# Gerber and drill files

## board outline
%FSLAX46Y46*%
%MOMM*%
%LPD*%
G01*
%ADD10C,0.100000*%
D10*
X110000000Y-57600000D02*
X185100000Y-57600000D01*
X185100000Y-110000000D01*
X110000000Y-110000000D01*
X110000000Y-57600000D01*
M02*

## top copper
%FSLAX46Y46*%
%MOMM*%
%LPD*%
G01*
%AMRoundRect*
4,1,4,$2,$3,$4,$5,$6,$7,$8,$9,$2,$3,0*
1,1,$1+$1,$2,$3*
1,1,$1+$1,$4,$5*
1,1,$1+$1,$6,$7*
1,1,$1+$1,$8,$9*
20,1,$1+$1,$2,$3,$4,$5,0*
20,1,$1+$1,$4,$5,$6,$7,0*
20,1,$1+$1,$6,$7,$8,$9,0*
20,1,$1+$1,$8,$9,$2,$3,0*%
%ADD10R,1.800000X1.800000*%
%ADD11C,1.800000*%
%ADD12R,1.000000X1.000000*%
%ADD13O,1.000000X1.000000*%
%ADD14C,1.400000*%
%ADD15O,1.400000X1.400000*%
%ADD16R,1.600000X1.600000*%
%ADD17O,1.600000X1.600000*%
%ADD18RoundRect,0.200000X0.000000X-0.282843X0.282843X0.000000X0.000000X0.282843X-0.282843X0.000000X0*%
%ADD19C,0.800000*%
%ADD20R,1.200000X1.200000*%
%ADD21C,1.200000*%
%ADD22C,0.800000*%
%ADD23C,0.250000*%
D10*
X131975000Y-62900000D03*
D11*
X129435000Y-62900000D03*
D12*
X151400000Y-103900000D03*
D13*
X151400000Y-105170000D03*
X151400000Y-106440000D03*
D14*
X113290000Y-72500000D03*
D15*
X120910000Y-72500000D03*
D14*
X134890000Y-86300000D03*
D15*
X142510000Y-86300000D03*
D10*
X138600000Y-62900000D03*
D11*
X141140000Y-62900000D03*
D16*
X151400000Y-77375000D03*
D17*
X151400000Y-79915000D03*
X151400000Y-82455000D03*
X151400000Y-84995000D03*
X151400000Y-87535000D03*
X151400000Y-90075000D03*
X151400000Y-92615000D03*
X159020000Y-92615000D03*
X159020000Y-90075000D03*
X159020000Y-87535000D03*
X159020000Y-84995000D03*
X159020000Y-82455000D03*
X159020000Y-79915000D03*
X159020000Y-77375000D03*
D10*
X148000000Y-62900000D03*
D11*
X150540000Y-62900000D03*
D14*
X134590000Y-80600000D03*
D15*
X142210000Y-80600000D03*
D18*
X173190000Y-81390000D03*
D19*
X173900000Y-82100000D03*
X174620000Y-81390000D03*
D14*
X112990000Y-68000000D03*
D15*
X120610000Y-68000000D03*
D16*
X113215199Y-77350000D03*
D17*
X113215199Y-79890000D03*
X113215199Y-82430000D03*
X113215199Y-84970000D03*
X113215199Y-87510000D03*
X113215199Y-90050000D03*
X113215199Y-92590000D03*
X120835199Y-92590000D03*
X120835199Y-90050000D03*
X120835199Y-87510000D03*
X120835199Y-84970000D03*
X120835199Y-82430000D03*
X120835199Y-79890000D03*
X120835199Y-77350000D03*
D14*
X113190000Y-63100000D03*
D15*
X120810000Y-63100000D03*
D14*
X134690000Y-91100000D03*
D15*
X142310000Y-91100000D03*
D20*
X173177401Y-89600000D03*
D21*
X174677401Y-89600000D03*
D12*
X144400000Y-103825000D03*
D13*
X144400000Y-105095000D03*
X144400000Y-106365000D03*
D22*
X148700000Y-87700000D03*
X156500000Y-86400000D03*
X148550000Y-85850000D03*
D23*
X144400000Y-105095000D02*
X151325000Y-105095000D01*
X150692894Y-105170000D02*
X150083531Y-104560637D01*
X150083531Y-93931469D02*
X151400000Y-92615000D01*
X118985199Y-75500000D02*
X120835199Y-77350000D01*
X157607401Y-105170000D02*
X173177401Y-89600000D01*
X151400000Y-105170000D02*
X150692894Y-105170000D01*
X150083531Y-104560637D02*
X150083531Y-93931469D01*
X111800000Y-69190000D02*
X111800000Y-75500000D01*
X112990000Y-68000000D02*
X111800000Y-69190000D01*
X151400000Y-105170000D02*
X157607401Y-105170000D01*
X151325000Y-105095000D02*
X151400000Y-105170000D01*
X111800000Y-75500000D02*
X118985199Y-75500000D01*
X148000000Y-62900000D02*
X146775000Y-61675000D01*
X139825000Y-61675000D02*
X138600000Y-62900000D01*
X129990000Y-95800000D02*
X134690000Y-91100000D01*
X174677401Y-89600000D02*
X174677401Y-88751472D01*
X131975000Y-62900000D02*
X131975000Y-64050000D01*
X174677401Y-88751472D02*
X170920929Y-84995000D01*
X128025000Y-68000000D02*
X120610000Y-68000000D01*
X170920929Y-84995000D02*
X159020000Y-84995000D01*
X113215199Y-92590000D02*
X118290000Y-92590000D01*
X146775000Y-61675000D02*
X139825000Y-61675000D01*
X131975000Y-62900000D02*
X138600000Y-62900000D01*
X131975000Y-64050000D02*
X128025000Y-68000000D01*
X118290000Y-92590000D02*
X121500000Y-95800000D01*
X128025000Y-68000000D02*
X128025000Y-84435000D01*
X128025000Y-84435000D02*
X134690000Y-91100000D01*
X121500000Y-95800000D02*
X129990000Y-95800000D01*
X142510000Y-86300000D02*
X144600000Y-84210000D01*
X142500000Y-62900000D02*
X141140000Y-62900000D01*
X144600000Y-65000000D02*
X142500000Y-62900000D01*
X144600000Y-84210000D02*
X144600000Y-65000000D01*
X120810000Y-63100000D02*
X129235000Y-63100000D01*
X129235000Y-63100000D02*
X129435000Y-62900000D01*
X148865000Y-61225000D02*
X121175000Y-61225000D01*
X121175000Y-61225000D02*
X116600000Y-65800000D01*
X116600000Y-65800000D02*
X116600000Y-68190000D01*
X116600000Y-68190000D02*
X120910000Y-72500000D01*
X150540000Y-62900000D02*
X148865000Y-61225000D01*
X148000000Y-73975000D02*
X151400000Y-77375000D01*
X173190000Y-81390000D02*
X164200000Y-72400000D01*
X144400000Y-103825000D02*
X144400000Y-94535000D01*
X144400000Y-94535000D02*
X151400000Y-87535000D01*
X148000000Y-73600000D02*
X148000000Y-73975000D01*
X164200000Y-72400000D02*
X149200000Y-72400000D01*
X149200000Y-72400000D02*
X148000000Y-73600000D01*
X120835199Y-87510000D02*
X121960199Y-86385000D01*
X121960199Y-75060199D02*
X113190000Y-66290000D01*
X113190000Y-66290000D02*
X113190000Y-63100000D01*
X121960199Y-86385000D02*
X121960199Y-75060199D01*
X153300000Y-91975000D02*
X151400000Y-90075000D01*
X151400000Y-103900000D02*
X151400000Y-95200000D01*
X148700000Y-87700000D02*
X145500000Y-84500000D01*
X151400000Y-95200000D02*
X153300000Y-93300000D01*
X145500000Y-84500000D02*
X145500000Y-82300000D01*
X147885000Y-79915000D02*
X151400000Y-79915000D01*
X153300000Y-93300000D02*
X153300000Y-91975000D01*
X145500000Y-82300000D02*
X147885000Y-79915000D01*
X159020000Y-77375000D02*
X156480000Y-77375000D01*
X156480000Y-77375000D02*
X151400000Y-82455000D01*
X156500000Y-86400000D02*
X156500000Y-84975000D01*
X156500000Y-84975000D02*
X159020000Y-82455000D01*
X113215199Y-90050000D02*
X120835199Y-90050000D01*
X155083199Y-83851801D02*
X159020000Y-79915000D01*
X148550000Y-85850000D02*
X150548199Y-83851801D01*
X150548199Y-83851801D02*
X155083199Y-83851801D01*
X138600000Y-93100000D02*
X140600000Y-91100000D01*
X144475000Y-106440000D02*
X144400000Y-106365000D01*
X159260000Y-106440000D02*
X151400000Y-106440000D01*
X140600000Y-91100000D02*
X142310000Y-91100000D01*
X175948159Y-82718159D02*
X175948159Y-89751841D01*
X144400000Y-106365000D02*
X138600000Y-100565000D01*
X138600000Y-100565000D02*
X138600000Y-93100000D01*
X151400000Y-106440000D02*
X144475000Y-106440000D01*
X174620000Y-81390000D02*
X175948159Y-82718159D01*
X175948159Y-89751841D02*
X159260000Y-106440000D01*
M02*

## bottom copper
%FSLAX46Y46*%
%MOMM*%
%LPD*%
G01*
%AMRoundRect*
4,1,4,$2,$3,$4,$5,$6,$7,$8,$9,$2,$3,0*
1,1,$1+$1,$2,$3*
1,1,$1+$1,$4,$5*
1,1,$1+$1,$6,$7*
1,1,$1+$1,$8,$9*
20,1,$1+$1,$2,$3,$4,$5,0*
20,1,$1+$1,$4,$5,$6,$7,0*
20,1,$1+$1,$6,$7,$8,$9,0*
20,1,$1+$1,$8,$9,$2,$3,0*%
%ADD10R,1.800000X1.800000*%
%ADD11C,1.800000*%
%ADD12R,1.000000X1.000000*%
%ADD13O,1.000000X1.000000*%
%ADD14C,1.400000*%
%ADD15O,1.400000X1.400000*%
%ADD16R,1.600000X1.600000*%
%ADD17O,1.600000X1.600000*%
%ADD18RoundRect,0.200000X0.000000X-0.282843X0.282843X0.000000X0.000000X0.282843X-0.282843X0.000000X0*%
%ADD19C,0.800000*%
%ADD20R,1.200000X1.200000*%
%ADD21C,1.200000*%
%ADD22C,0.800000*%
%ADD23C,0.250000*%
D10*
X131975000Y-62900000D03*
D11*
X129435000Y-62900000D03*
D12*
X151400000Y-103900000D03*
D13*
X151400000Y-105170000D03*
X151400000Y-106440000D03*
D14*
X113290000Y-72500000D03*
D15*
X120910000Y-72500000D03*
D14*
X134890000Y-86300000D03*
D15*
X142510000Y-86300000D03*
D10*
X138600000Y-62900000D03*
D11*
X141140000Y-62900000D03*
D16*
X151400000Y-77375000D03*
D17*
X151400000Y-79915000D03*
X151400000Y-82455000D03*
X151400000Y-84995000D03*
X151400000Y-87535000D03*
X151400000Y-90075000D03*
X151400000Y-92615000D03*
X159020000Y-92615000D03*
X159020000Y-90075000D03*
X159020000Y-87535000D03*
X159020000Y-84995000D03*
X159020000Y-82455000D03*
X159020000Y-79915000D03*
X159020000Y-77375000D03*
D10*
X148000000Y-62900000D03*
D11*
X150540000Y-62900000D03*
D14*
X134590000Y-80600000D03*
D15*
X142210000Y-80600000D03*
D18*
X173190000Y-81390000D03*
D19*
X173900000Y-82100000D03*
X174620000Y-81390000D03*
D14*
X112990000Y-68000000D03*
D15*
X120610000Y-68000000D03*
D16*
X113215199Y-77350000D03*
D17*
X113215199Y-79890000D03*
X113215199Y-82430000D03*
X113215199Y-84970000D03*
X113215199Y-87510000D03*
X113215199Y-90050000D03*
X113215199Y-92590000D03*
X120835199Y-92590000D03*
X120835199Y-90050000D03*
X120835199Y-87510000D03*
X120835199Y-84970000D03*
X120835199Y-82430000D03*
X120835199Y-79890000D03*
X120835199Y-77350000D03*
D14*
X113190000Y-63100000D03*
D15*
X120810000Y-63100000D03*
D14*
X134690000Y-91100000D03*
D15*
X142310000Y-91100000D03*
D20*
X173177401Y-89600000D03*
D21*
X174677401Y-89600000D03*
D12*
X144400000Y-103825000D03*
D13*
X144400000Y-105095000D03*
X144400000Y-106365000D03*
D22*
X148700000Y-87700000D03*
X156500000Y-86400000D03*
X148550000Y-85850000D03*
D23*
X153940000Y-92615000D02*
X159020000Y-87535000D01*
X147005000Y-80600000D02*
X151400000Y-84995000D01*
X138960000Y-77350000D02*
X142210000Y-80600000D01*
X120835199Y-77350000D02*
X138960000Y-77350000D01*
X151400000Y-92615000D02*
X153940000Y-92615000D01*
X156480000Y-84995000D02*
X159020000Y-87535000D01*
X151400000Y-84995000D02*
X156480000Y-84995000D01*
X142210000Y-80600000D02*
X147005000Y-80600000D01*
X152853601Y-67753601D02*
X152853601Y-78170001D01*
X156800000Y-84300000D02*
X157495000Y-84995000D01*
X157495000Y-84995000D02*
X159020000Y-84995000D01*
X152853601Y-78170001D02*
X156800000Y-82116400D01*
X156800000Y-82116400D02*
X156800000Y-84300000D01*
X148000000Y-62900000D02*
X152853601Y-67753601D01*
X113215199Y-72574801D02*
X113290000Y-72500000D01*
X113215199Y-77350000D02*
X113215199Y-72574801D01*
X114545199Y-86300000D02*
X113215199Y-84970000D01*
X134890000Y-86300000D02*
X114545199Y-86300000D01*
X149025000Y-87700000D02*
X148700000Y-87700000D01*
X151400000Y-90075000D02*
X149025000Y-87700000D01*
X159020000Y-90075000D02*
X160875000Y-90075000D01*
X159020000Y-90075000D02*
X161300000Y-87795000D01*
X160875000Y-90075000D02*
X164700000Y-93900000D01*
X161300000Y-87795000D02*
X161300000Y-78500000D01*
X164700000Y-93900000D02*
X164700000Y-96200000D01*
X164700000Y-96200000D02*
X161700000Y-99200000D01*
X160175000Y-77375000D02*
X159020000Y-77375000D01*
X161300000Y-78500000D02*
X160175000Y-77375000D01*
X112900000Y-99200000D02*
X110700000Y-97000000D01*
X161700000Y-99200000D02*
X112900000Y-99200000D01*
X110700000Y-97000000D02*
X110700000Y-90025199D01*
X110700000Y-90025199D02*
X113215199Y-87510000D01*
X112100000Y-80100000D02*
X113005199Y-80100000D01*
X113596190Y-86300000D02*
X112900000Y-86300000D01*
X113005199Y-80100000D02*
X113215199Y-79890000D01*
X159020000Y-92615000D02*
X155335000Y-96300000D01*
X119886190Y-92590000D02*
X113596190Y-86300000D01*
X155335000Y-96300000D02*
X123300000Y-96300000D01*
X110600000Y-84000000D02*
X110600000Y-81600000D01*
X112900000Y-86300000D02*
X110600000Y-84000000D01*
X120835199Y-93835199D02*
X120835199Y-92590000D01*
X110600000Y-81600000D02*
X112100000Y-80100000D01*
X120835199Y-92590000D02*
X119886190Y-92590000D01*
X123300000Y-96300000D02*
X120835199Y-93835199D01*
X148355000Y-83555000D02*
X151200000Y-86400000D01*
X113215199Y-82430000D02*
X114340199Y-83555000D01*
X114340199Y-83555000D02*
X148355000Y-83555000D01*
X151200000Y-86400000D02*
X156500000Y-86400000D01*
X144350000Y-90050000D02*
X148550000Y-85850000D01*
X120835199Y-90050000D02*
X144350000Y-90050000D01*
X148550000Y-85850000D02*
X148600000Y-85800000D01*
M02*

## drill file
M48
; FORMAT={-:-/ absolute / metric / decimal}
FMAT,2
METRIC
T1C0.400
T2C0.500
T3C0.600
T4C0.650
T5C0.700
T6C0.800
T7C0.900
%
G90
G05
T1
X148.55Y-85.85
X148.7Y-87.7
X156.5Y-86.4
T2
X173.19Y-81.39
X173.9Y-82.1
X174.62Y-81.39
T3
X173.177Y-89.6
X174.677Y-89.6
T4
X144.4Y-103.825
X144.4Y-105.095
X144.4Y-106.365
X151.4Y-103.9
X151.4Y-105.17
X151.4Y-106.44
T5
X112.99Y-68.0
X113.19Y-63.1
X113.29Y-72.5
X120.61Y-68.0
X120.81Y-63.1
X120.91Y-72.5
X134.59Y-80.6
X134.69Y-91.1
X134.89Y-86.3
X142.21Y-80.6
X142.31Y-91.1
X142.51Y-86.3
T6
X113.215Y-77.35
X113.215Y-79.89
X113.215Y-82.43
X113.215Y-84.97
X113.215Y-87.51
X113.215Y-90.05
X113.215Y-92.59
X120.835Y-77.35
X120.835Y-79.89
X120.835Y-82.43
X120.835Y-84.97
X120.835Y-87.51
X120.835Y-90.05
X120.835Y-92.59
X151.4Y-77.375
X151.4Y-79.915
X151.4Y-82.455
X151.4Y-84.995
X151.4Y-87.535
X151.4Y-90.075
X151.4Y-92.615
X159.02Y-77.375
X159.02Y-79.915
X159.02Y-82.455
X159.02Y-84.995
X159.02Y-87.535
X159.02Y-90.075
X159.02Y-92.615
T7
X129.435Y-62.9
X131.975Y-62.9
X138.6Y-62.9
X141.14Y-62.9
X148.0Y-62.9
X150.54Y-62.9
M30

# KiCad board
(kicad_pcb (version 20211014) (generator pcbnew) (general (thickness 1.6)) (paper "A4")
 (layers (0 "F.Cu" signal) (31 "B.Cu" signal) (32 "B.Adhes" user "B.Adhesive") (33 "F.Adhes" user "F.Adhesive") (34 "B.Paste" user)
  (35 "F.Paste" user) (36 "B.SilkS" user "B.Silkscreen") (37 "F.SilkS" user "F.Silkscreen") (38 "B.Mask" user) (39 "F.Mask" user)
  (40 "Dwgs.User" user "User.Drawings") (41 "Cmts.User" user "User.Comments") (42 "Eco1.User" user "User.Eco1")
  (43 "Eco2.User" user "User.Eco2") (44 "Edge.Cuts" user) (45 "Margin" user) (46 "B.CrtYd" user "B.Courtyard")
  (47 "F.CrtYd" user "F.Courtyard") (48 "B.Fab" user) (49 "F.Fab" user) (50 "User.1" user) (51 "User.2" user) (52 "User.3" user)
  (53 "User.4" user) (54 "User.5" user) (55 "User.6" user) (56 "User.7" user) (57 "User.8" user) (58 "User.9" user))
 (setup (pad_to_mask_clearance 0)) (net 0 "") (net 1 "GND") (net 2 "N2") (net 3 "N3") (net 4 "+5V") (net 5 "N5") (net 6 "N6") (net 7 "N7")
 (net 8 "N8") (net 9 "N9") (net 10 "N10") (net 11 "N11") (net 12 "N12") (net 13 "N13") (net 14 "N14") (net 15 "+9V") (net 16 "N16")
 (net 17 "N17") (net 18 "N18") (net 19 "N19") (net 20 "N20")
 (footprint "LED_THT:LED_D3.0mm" (layer "F.Cu") (at 131.975 62.9 180)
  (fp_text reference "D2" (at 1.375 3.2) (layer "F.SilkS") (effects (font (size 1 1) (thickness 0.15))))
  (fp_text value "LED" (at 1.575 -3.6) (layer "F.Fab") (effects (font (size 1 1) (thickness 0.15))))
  (pad "1" thru_hole rect (at 0 0 180) (size 1.8 1.8) (drill 0.9) (layers *.Cu *.Mask) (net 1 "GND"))
  (pad "2" thru_hole circle (at 2.54 0 180) (size 1.8 1.8) (drill 0.9) (layers *.Cu *.Mask) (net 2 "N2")))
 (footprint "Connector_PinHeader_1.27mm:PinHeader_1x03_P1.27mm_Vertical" (layer "F.Cu") (at 151.4 103.9)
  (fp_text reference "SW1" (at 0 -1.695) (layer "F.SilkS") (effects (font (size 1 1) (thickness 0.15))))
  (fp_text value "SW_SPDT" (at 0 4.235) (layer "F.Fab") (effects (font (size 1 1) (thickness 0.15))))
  (pad "1" thru_hole rect (at 0 0) (size 1 1) (drill 0.65) (layers *.Cu *.Mask) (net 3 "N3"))
  (pad "2" thru_hole oval (at 0 1.27) (size 1 1) (drill 0.65) (layers *.Cu *.Mask) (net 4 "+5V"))
  (pad "3" thru_hole oval (at 0 2.54) (size 1 1) (drill 0.65) (layers *.Cu *.Mask) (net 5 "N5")))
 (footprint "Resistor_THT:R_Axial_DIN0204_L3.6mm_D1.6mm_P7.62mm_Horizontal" (layer "F.Cu") (at 113.29 72.5)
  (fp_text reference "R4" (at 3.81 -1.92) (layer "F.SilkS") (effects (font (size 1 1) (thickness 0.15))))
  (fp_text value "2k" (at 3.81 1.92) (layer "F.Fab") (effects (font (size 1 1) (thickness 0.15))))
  (pad "1" thru_hole circle (at 0 0) (size 1.4 1.4) (drill 0.7) (layers *.Cu *.Mask) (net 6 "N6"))
  (pad "2" thru_hole oval (at 7.62 0) (size 1.4 1.4) (drill 0.7) (layers *.Cu *.Mask) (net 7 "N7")))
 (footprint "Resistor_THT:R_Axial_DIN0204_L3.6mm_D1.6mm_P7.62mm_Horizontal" (layer "F.Cu") (at 134.89 86.3)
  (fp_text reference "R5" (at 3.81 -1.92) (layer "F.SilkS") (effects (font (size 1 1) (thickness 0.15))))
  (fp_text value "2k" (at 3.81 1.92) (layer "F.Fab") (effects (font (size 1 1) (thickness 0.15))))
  (pad "1" thru_hole circle (at 0 0) (size 1.4 1.4) (drill 0.7) (layers *.Cu *.Mask) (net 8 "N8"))
  (pad "2" thru_hole oval (at 7.62 0) (size 1.4 1.4) (drill 0.7) (layers *.Cu *.Mask) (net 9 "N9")))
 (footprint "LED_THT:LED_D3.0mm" (layer "F.Cu") (at 138.6 62.9)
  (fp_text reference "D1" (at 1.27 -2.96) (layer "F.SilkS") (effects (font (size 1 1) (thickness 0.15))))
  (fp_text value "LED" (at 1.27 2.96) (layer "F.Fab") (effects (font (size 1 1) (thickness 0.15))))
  (pad "1" thru_hole rect (at 0 0) (size 1.8 1.8) (drill 0.9) (layers *.Cu *.Mask) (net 1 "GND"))
  (pad "2" thru_hole circle (at 2.54 0) (size 1.8 1.8) (drill 0.9) (layers *.Cu *.Mask) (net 9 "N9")))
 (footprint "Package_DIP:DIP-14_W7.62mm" (layer "F.Cu") (at 151.4 77.375)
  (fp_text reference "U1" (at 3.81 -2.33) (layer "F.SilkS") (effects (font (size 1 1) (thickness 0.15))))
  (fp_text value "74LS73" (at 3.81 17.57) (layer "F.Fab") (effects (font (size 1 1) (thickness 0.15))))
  (pad "1" thru_hole rect (at 0 0) (size 1.6 1.6) (drill 0.8) (layers *.Cu *.Mask) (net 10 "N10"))
  (pad "2" thru_hole oval (at 0 2.54) (size 1.6 1.6) (drill 0.8) (layers *.Cu *.Mask) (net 3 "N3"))
  (pad "3" thru_hole oval (at 0 5.08) (size 1.6 1.6) (drill 0.8) (layers *.Cu *.Mask) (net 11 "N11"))
  (pad "4" thru_hole oval (at 0 7.62) (size 1.6 1.6) (drill 0.8) (layers *.Cu *.Mask) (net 4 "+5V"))
  (pad "5" thru_hole oval (at 0 10.16) (size 1.6 1.6) (drill 0.8) (layers *.Cu *.Mask) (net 10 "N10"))
  (pad "6" thru_hole oval (at 0 12.7) (size 1.6 1.6) (drill 0.8) (layers *.Cu *.Mask) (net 3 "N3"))
  (pad "7" thru_hole oval (at 0 15.24) (size 1.6 1.6) (drill 0.8) (layers *.Cu *.Mask) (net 4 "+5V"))
  (pad "8" thru_hole oval (at 7.62 15.24) (size 1.6 1.6) (drill 0.8) (layers *.Cu *.Mask) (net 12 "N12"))
  (pad "9" thru_hole oval (at 7.62 12.7) (size 1.6 1.6) (drill 0.8) (layers *.Cu *.Mask) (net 11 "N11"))
  (pad "10" thru_hole oval (at 7.62 10.16) (size 1.6 1.6) (drill 0.8) (layers *.Cu *.Mask) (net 4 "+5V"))
  (pad "11" thru_hole oval (at 7.62 7.62) (size 1.6 1.6) (drill 0.8) (layers *.Cu *.Mask) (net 1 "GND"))
  (pad "12" thru_hole oval (at 7.62 5.08) (size 1.6 1.6) (drill 0.8) (layers *.Cu *.Mask) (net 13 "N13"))
  (pad "13" thru_hole oval (at 7.62 2.54) (size 1.6 1.6) (drill 0.8) (layers *.Cu *.Mask) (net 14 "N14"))
  (pad "14" thru_hole oval (at 7.62 0) (size 1.6 1.6) (drill 0.8) (layers *.Cu *.Mask) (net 11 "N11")))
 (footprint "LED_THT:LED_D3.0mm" (layer "F.Cu") (at 148 62.9)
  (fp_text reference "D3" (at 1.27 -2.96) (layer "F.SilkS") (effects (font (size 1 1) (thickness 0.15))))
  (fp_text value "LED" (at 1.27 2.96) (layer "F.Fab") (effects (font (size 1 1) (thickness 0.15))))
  (pad "1" thru_hole rect (at 0 0) (size 1.8 1.8) (drill 0.9) (layers *.Cu *.Mask) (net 1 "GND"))
  (pad "2" thru_hole circle (at 2.54 0) (size 1.8 1.8) (drill 0.9) (layers *.Cu *.Mask) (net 7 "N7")))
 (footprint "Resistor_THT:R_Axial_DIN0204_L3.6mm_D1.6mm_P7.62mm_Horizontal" (layer "F.Cu") (at 134.59 80.6)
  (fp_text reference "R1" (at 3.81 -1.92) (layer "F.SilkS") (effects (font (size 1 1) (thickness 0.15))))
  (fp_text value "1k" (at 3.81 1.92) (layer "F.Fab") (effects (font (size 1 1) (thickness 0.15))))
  (pad "1" thru_hole circle (at 0 0) (size 1.4 1.4) (drill 0.7) (layers *.Cu *.Mask) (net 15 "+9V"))
  (pad "2" thru_hole oval (at 7.62 0) (size 1.4 1.4) (drill 0.7) (layers *.Cu *.Mask) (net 4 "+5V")))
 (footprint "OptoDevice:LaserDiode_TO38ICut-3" (layer "F.Cu") (at 173.19 81.39)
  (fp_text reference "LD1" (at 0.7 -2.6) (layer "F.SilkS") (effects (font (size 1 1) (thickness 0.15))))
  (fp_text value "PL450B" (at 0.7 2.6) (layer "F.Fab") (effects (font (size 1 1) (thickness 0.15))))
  (pad "1" thru_hole roundrect (at 0 0 45) (size 0.8 0.8) (drill 0.5) (layers *.Cu *.Mask) (roundrect_rratio 0.25) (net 10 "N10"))
  (pad "2" thru_hole circle (at 0.71 0.71) (size 0.8 0.8) (drill 0.5) (layers *.Cu *.Mask) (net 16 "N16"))
  (pad "3" thru_hole circle (at 1.43 0) (size 0.8 0.8) (drill 0.5) (layers *.Cu *.Mask) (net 5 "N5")))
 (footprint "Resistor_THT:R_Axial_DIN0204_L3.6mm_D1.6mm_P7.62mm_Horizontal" (layer "F.Cu") (at 112.99 68)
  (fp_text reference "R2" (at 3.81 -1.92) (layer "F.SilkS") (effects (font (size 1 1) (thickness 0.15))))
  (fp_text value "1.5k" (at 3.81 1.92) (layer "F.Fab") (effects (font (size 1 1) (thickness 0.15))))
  (pad "1" thru_hole circle (at 0 0) (size 1.4 1.4) (drill 0.7) (layers *.Cu *.Mask) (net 4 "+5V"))
  (pad "2" thru_hole oval (at 7.62 0) (size 1.4 1.4) (drill 0.7) (layers *.Cu *.Mask) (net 1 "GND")))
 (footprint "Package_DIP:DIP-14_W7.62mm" (layer "F.Cu") (at 113.215199 77.35)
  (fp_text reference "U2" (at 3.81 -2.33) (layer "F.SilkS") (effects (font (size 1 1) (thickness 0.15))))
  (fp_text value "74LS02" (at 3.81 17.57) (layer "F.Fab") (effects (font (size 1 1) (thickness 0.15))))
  (pad "1" thru_hole rect (at 0 0) (size 1.6 1.6) (drill 0.8) (layers *.Cu *.Mask) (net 6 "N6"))
  (pad "2" thru_hole oval (at 0 2.54) (size 1.6 1.6) (drill 0.8) (layers *.Cu *.Mask) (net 12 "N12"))
  (pad "3" thru_hole oval (at 0 5.08) (size 1.6 1.6) (drill 0.8) (layers *.Cu *.Mask) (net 13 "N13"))
  (pad "4" thru_hole oval (at 0 7.62) (size 1.6 1.6) (drill 0.8) (layers *.Cu *.Mask) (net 8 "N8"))
  (pad "5" thru_hole oval (at 0 10.16) (size 1.6 1.6) (drill 0.8) (layers *.Cu *.Mask) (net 11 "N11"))
  (pad "6" thru_hole oval (at 0 12.7) (size 1.6 1.6) (drill 0.8) (layers *.Cu *.Mask) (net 14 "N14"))
  (pad "7" thru_hole oval (at 0 15.24) (size 1.6 1.6) (drill 0.8) (layers *.Cu *.Mask) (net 1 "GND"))
  (pad "8" thru_hole oval (at 7.62 15.24) (size 1.6 1.6) (drill 0.8) (layers *.Cu *.Mask) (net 12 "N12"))
  (pad "9" thru_hole oval (at 7.62 12.7) (size 1.6 1.6) (drill 0.8) (layers *.Cu *.Mask) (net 14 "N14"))
  (pad "10" thru_hole oval (at 7.62 10.16) (size 1.6 1.6) (drill 0.8) (layers *.Cu *.Mask) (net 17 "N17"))
  (pad "11" thru_hole oval (at 7.62 7.62) (size 1.6 1.6) (drill 0.8) (layers *.Cu *.Mask) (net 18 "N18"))
  (pad "12" thru_hole oval (at 7.62 5.08) (size 1.6 1.6) (drill 0.8) (layers *.Cu *.Mask) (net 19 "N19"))
  (pad "13" thru_hole oval (at 7.62 2.54) (size 1.6 1.6) (drill 0.8) (layers *.Cu *.Mask) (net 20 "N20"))
  (pad "14" thru_hole oval (at 7.62 0) (size 1.6 1.6) (drill 0.8) (layers *.Cu *.Mask) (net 4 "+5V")))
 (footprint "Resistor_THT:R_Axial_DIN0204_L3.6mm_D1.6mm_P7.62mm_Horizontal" (layer "F.Cu") (at 113.19 63.1)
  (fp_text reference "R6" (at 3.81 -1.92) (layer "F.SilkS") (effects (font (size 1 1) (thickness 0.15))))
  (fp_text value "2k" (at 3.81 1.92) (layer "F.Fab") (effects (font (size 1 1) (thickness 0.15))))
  (pad "1" thru_hole circle (at 0 0) (size 1.4 1.4) (drill 0.7) (layers *.Cu *.Mask) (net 17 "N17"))
  (pad "2" thru_hole oval (at 7.62 0) (size 1.4 1.4) (drill 0.7) (layers *.Cu *.Mask) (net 2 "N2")))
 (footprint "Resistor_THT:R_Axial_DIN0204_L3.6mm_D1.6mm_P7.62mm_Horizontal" (layer "F.Cu") (at 134.69 91.1)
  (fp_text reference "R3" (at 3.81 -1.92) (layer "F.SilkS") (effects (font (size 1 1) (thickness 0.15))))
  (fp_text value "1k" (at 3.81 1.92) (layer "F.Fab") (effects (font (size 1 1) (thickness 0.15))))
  (pad "1" thru_hole circle (at 0 0) (size 1.4 1.4) (drill 0.7) (layers *.Cu *.Mask) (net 1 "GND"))
  (pad "2" thru_hole oval (at 7.62 0) (size 1.4 1.4) (drill 0.7) (layers *.Cu *.Mask) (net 5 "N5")))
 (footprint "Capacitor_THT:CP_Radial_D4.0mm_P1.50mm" (layer "F.Cu") (at 173.177401 89.6)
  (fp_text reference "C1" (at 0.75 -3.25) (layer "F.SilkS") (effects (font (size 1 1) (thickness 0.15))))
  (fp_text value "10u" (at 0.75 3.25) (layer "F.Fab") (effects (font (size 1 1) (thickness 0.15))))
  (pad "1" thru_hole rect (at 0 0) (size 1.2 1.2) (drill 0.6) (layers *.Cu *.Mask) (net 4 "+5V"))
  (pad "2" thru_hole circle (at 1.5 0) (size 1.2 1.2) (drill 0.6) (layers *.Cu *.Mask) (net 1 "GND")))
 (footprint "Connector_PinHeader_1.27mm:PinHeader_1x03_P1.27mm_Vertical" (layer "F.Cu") (at 144.4 103.825)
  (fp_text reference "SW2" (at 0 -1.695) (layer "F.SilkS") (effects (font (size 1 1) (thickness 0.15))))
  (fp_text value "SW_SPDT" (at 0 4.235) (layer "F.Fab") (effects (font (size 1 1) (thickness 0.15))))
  (pad "1" thru_hole rect (at 0 0) (size 1 1) (drill 0.65) (layers *.Cu *.Mask) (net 10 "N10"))
  (pad "2" thru_hole oval (at 0 1.27) (size 1 1) (drill 0.65) (layers *.Cu *.Mask) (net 4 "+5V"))
  (pad "3" thru_hole oval (at 0 2.54) (size 1 1) (drill 0.65) (layers *.Cu *.Mask) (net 5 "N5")))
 (gr_rect (start 110 57.6) (end 185.1 110) (layer "Edge.Cuts") (width 0.1) (fill none))
 (segment (start 144.4 105.095) (end 151.325 105.095) (width 0.25) (layer "F.Cu") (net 4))
 (segment (start 150.692894 105.17) (end 150.083531 104.560637) (width 0.25) (layer "F.Cu") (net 4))
 (segment (start 150.083531 93.931469) (end 151.4 92.615) (width 0.25) (layer "F.Cu") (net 4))
 (segment (start 118.985199 75.5) (end 120.835199 77.35) (width 0.25) (layer "F.Cu") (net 4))
 (segment (start 157.607401 105.17) (end 173.177401 89.6) (width 0.25) (layer "F.Cu") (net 4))
 (segment (start 151.4 105.17) (end 150.692894 105.17) (width 0.25) (layer "F.Cu") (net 4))
 (segment (start 150.083531 104.560637) (end 150.083531 93.931469) (width 0.25) (layer "F.Cu") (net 4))
 (segment (start 111.8 69.19) (end 111.8 75.5) (width 0.25) (layer "F.Cu") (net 4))
 (segment (start 112.99 68) (end 111.8 69.19) (width 0.25) (layer "F.Cu") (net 4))
 (segment (start 151.4 105.17) (end 157.607401 105.17) (width 0.25) (layer "F.Cu") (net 4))
 (segment (start 151.325 105.095) (end 151.4 105.17) (width 0.25) (layer "F.Cu") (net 4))
 (segment (start 111.8 75.5) (end 118.985199 75.5) (width 0.25) (layer "F.Cu") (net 4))
 (segment (start 153.94 92.615) (end 159.02 87.535) (width 0.25) (layer "B.Cu") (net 4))
 (segment (start 147.005 80.6) (end 151.4 84.995) (width 0.25) (layer "B.Cu") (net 4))
 (segment (start 138.96 77.35) (end 142.21 80.6) (width 0.25) (layer "B.Cu") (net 4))
 (segment (start 120.835199 77.35) (end 138.96 77.35) (width 0.25) (layer "B.Cu") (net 4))
 (segment (start 151.4 92.615) (end 153.94 92.615) (width 0.25) (layer "B.Cu") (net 4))
 (segment (start 156.48 84.995) (end 159.02 87.535) (width 0.25) (layer "B.Cu") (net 4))
 (segment (start 151.4 84.995) (end 156.48 84.995) (width 0.25) (layer "B.Cu") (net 4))
 (segment (start 142.21 80.6) (end 147.005 80.6) (width 0.25) (layer "B.Cu") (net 4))
 (segment (start 148 62.9) (end 146.775 61.675) (width 0.25) (layer "F.Cu") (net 1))
 (segment (start 139.825 61.675) (end 138.6 62.9) (width 0.25) (layer "F.Cu") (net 1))
 (segment (start 129.99 95.8) (end 134.69 91.1) (width 0.25) (layer "F.Cu") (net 1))
 (segment (start 174.677401 89.6) (end 174.677401 88.751472) (width 0.25) (layer "F.Cu") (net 1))
 (segment (start 131.975 62.9) (end 131.975 64.05) (width 0.25) (layer "F.Cu") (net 1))
 (segment (start 174.677401 88.751472) (end 170.920929 84.995) (width 0.25) (layer "F.Cu") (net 1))
 (segment (start 128.025 68) (end 120.61 68) (width 0.25) (layer "F.Cu") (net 1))
 (segment (start 170.920929 84.995) (end 159.02 84.995) (width 0.25) (layer "F.Cu") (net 1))
 (segment (start 113.215199 92.59) (end 118.29 92.59) (width 0.25) (layer "F.Cu") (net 1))
 (segment (start 146.775 61.675) (end 139.825 61.675) (width 0.25) (layer "F.Cu") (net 1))
 (segment (start 131.975 62.9) (end 138.6 62.9) (width 0.25) (layer "F.Cu") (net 1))
 (segment (start 131.975 64.05) (end 128.025 68) (width 0.25) (layer "F.Cu") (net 1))
 (segment (start 118.29 92.59) (end 121.5 95.8) (width 0.25) (layer "F.Cu") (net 1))
 (segment (start 128.025 68) (end 128.025 84.435) (width 0.25) (layer "F.Cu") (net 1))
 (segment (start 128.025 84.435) (end 134.69 91.1) (width 0.25) (layer "F.Cu") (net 1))
 (segment (start 121.5 95.8) (end 129.99 95.8) (width 0.25) (layer "F.Cu") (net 1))
 (segment (start 152.853601 67.753601) (end 152.853601 78.170001) (width 0.25) (layer "B.Cu") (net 1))
 (segment (start 156.8 84.3) (end 157.495 84.995) (width 0.25) (layer "B.Cu") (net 1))
 (segment (start 157.495 84.995) (end 159.02 84.995) (width 0.25) (layer "B.Cu") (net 1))
 (segment (start 152.853601 78.170001) (end 156.8 82.1164) (width 0.25) (layer "B.Cu") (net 1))
 (segment (start 156.8 82.1164) (end 156.8 84.3) (width 0.25) (layer "B.Cu") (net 1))
 (segment (start 148 62.9) (end 152.853601 67.753601) (width 0.25) (layer "B.Cu") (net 1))
 (segment (start 142.51 86.3) (end 144.6 84.21) (width 0.25) (layer "F.Cu") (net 9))
 (segment (start 142.5 62.9) (end 141.14 62.9) (width 0.25) (layer "F.Cu") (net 9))
 (segment (start 144.6 65) (end 142.5 62.9) (width 0.25) (layer "F.Cu") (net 9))
 (segment (start 144.6 84.21) (end 144.6 65) (width 0.25) (layer "F.Cu") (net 9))
 (segment (start 120.81 63.1) (end 129.235 63.1) (width 0.25) (layer "F.Cu") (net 2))
 (segment (start 129.235 63.1) (end 129.435 62.9) (width 0.25) (layer "F.Cu") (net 2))
 (segment (start 148.865 61.225) (end 121.175 61.225) (width 0.25) (layer "F.Cu") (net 7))
 (segment (start 121.175 61.225) (end 116.6 65.8) (width 0.25) (layer "F.Cu") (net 7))
 (segment (start 116.6 65.8) (end 116.6 68.19) (width 0.25) (layer "F.Cu") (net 7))
 (segment (start 116.6 68.19) (end 120.91 72.5) (width 0.25) (layer "F.Cu") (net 7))
 (segment (start 150.54 62.9) (end 148.865 61.225) (width 0.25) (layer "F.Cu") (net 7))
 (segment (start 148 73.975) (end 151.4 77.375) (width 0.25) (layer "F.Cu") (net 10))
 (segment (start 173.19 81.39) (end 164.2 72.4) (width 0.25) (layer "F.Cu") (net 10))
 (segment (start 144.4 103.825) (end 144.4 94.535) (width 0.25) (layer "F.Cu") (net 10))
 (segment (start 144.4 94.535) (end 151.4 87.535) (width 0.25) (layer "F.Cu") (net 10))
 (segment (start 148 73.6) (end 148 73.975) (width 0.25) (layer "F.Cu") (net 10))
 (segment (start 164.2 72.4) (end 149.2 72.4) (width 0.25) (layer "F.Cu") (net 10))
 (segment (start 149.2 72.4) (end 148 73.6) (width 0.25) (layer "F.Cu") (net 10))
 (segment (start 113.215199 72.574801) (end 113.29 72.5) (width 0.25) (layer "B.Cu") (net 6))
 (segment (start 113.215199 77.35) (end 113.215199 72.574801) (width 0.25) (layer "B.Cu") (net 6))
 (segment (start 114.545199 86.3) (end 113.215199 84.97) (width 0.25) (layer "B.Cu") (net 8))
 (segment (start 134.89 86.3) (end 114.545199 86.3) (width 0.25) (layer "B.Cu") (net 8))
 (segment (start 120.835199 87.51) (end 121.960199 86.385) (width 0.25) (layer "F.Cu") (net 17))
 (segment (start 121.960199 75.060199) (end 113.19 66.29) (width 0.25) (layer "F.Cu") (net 17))
 (segment (start 113.19 66.29) (end 113.19 63.1) (width 0.25) (layer "F.Cu") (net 17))
 (segment (start 121.960199 86.385) (end 121.960199 75.060199) (width 0.25) (layer "F.Cu") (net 17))
 (segment (start 153.3 91.975) (end 151.4 90.075) (width 0.25) (layer "F.Cu") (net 3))
 (segment (start 151.4 103.9) (end 151.4 95.2) (width 0.25) (layer "F.Cu") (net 3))
 (segment (start 148.7 87.7) (end 145.5 84.5) (width 0.25) (layer "F.Cu") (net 3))
 (segment (start 151.4 95.2) (end 153.3 93.3) (width 0.25) (layer "F.Cu") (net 3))
 (segment (start 145.5 84.5) (end 145.5 82.3) (width 0.25) (layer "F.Cu") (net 3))
 (segment (start 147.885 79.915) (end 151.4 79.915) (width 0.25) (layer "F.Cu") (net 3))
 (segment (start 153.3 93.3) (end 153.3 91.975) (width 0.25) (layer "F.Cu") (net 3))
 (segment (start 145.5 82.3) (end 147.885 79.915) (width 0.25) (layer "F.Cu") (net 3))
 (via (at 148.7 87.7) (size 0.8) (drill 0.4) (layers "F.Cu" "B.Cu") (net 3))
 (segment (start 149.025 87.7) (end 148.7 87.7) (width 0.25) (layer "B.Cu") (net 3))
 (segment (start 151.4 90.075) (end 149.025 87.7) (width 0.25) (layer "B.Cu") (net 3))
 (segment (start 159.02 77.375) (end 156.48 77.375) (width 0.25) (layer "F.Cu") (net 11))
 (segment (start 156.48 77.375) (end 151.4 82.455) (width 0.25) (layer "F.Cu") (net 11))
 (segment (start 159.02 90.075) (end 160.875 90.075) (width 0.25) (layer "B.Cu") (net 11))
 (segment (start 159.02 90.075) (end 161.3 87.795) (width 0.25) (layer "B.Cu") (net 11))
 (segment (start 160.875 90.075) (end 164.7 93.9) (width 0.25) (layer "B.Cu") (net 11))
 (segment (start 161.3 87.795) (end 161.3 78.5) (width 0.25) (layer "B.Cu") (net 11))
 (segment (start 164.7 93.9) (end 164.7 96.2) (width 0.25) (layer "B.Cu") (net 11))
 (segment (start 164.7 96.2) (end 161.7 99.2) (width 0.25) (layer "B.Cu") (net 11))
 (segment (start 160.175 77.375) (end 159.02 77.375) (width 0.25) (layer "B.Cu") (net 11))
 (segment (start 161.3 78.5) (end 160.175 77.375) (width 0.25) (layer "B.Cu") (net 11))
 (segment (start 112.9 99.2) (end 110.7 97) (width 0.25) (layer "B.Cu") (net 11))
 (segment (start 161.7 99.2) (end 112.9 99.2) (width 0.25) (layer "B.Cu") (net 11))
 (segment (start 110.7 97) (end 110.7 90.025199) (width 0.25) (layer "B.Cu") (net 11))
 (segment (start 110.7 90.025199) (end 113.215199 87.51) (width 0.25) (layer "B.Cu") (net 11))
 (segment (start 112.1 80.1) (end 113.005199 80.1) (width 0.25) (layer "B.Cu") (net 12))
 (segment (start 113.59619 86.3) (end 112.9 86.3) (width 0.25) (layer "B.Cu") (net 12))
 (segment (start 113.005199 80.1) (end 113.215199 79.89) (width 0.25) (layer "B.Cu") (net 12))
 (segment (start 159.02 92.615) (end 155.335 96.3) (width 0.25) (layer "B.Cu") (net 12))
 (segment (start 119.88619 92.59) (end 113.59619 86.3) (width 0.25) (layer "B.Cu") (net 12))
 (segment (start 155.335 96.3) (end 123.3 96.3) (width 0.25) (layer "B.Cu") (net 12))
 (segment (start 110.6 84) (end 110.6 81.6) (width 0.25) (layer "B.Cu") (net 12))
 (segment (start 112.9 86.3) (end 110.6 84) (width 0.25) (layer "B.Cu") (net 12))
 (segment (start 120.835199 93.835199) (end 120.835199 92.59) (width 0.25) (layer "B.Cu") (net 12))
 (segment (start 110.6 81.6) (end 112.1 80.1) (width 0.25) (layer "B.Cu") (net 12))
 (segment (start 120.835199 92.59) (end 119.88619 92.59) (width 0.25) (layer "B.Cu") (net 12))
 (segment (start 123.3 96.3) (end 120.835199 93.835199) (width 0.25) (layer "B.Cu") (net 12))
 (segment (start 156.5 86.4) (end 156.5 84.975) (width 0.25) (layer "F.Cu") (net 13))
 (segment (start 156.5 84.975) (end 159.02 82.455) (width 0.25) (layer "F.Cu") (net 13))
 (via (at 156.5 86.4) (size 0.8) (drill 0.4) (layers "F.Cu" "B.Cu") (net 13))
 (segment (start 148.355 83.555) (end 151.2 86.4) (width 0.25) (layer "B.Cu") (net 13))
 (segment (start 113.215199 82.43) (end 114.340199 83.555) (width 0.25) (layer "B.Cu") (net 13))
 (segment (start 114.340199 83.555) (end 148.355 83.555) (width 0.25) (layer "B.Cu") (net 13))
 (segment (start 151.2 86.4) (end 156.5 86.4) (width 0.25) (layer "B.Cu") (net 13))
 (segment (start 113.215199 90.05) (end 120.835199 90.05) (width 0.25) (layer "F.Cu") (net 14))
 (segment (start 155.083199 83.851801) (end 159.02 79.915) (width 0.25) (layer "F.Cu") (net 14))
 (segment (start 148.55 85.85) (end 150.548199 83.851801) (width 0.25) (layer "F.Cu") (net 14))
 (segment (start 150.548199 83.851801) (end 155.083199 83.851801) (width 0.25) (layer "F.Cu") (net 14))
 (via (at 148.55 85.85) (size 0.8) (drill 0.4) (layers "F.Cu" "B.Cu") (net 14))
 (segment (start 144.35 90.05) (end 148.55 85.85) (width 0.25) (layer "B.Cu") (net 14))
 (segment (start 120.835199 90.05) (end 144.35 90.05) (width 0.25) (layer "B.Cu") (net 14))
 (segment (start 148.55 85.85) (end 148.6 85.8) (width 0.25) (layer "B.Cu") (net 14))
 (segment (start 138.6 93.1) (end 140.6 91.1) (width 0.25) (layer "F.Cu") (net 5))
 (segment (start 144.475 106.44) (end 144.4 106.365) (width 0.25) (layer "F.Cu") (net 5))
 (segment (start 159.26 106.44) (end 151.4 106.44) (width 0.25) (layer "F.Cu") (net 5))
 (segment (start 140.6 91.1) (end 142.31 91.1) (width 0.25) (layer "F.Cu") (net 5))
 (segment (start 175.948159 82.718159) (end 175.948159 89.751841) (width 0.25) (layer "F.Cu") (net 5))
 (segment (start 144.4 106.365) (end 138.6 100.565) (width 0.25) (layer "F.Cu") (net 5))
 (segment (start 138.6 100.565) (end 138.6 93.1) (width 0.25) (layer "F.Cu") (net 5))
 (segment (start 151.4 106.44) (end 144.475 106.44) (width 0.25) (layer "F.Cu") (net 5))
 (segment (start 174.62 81.39) (end 175.948159 82.718159) (width 0.25) (layer "F.Cu") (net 5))
 (segment (start 175.948159 89.751841) (end 159.26 106.44) (width 0.25) (layer "F.Cu") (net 5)))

